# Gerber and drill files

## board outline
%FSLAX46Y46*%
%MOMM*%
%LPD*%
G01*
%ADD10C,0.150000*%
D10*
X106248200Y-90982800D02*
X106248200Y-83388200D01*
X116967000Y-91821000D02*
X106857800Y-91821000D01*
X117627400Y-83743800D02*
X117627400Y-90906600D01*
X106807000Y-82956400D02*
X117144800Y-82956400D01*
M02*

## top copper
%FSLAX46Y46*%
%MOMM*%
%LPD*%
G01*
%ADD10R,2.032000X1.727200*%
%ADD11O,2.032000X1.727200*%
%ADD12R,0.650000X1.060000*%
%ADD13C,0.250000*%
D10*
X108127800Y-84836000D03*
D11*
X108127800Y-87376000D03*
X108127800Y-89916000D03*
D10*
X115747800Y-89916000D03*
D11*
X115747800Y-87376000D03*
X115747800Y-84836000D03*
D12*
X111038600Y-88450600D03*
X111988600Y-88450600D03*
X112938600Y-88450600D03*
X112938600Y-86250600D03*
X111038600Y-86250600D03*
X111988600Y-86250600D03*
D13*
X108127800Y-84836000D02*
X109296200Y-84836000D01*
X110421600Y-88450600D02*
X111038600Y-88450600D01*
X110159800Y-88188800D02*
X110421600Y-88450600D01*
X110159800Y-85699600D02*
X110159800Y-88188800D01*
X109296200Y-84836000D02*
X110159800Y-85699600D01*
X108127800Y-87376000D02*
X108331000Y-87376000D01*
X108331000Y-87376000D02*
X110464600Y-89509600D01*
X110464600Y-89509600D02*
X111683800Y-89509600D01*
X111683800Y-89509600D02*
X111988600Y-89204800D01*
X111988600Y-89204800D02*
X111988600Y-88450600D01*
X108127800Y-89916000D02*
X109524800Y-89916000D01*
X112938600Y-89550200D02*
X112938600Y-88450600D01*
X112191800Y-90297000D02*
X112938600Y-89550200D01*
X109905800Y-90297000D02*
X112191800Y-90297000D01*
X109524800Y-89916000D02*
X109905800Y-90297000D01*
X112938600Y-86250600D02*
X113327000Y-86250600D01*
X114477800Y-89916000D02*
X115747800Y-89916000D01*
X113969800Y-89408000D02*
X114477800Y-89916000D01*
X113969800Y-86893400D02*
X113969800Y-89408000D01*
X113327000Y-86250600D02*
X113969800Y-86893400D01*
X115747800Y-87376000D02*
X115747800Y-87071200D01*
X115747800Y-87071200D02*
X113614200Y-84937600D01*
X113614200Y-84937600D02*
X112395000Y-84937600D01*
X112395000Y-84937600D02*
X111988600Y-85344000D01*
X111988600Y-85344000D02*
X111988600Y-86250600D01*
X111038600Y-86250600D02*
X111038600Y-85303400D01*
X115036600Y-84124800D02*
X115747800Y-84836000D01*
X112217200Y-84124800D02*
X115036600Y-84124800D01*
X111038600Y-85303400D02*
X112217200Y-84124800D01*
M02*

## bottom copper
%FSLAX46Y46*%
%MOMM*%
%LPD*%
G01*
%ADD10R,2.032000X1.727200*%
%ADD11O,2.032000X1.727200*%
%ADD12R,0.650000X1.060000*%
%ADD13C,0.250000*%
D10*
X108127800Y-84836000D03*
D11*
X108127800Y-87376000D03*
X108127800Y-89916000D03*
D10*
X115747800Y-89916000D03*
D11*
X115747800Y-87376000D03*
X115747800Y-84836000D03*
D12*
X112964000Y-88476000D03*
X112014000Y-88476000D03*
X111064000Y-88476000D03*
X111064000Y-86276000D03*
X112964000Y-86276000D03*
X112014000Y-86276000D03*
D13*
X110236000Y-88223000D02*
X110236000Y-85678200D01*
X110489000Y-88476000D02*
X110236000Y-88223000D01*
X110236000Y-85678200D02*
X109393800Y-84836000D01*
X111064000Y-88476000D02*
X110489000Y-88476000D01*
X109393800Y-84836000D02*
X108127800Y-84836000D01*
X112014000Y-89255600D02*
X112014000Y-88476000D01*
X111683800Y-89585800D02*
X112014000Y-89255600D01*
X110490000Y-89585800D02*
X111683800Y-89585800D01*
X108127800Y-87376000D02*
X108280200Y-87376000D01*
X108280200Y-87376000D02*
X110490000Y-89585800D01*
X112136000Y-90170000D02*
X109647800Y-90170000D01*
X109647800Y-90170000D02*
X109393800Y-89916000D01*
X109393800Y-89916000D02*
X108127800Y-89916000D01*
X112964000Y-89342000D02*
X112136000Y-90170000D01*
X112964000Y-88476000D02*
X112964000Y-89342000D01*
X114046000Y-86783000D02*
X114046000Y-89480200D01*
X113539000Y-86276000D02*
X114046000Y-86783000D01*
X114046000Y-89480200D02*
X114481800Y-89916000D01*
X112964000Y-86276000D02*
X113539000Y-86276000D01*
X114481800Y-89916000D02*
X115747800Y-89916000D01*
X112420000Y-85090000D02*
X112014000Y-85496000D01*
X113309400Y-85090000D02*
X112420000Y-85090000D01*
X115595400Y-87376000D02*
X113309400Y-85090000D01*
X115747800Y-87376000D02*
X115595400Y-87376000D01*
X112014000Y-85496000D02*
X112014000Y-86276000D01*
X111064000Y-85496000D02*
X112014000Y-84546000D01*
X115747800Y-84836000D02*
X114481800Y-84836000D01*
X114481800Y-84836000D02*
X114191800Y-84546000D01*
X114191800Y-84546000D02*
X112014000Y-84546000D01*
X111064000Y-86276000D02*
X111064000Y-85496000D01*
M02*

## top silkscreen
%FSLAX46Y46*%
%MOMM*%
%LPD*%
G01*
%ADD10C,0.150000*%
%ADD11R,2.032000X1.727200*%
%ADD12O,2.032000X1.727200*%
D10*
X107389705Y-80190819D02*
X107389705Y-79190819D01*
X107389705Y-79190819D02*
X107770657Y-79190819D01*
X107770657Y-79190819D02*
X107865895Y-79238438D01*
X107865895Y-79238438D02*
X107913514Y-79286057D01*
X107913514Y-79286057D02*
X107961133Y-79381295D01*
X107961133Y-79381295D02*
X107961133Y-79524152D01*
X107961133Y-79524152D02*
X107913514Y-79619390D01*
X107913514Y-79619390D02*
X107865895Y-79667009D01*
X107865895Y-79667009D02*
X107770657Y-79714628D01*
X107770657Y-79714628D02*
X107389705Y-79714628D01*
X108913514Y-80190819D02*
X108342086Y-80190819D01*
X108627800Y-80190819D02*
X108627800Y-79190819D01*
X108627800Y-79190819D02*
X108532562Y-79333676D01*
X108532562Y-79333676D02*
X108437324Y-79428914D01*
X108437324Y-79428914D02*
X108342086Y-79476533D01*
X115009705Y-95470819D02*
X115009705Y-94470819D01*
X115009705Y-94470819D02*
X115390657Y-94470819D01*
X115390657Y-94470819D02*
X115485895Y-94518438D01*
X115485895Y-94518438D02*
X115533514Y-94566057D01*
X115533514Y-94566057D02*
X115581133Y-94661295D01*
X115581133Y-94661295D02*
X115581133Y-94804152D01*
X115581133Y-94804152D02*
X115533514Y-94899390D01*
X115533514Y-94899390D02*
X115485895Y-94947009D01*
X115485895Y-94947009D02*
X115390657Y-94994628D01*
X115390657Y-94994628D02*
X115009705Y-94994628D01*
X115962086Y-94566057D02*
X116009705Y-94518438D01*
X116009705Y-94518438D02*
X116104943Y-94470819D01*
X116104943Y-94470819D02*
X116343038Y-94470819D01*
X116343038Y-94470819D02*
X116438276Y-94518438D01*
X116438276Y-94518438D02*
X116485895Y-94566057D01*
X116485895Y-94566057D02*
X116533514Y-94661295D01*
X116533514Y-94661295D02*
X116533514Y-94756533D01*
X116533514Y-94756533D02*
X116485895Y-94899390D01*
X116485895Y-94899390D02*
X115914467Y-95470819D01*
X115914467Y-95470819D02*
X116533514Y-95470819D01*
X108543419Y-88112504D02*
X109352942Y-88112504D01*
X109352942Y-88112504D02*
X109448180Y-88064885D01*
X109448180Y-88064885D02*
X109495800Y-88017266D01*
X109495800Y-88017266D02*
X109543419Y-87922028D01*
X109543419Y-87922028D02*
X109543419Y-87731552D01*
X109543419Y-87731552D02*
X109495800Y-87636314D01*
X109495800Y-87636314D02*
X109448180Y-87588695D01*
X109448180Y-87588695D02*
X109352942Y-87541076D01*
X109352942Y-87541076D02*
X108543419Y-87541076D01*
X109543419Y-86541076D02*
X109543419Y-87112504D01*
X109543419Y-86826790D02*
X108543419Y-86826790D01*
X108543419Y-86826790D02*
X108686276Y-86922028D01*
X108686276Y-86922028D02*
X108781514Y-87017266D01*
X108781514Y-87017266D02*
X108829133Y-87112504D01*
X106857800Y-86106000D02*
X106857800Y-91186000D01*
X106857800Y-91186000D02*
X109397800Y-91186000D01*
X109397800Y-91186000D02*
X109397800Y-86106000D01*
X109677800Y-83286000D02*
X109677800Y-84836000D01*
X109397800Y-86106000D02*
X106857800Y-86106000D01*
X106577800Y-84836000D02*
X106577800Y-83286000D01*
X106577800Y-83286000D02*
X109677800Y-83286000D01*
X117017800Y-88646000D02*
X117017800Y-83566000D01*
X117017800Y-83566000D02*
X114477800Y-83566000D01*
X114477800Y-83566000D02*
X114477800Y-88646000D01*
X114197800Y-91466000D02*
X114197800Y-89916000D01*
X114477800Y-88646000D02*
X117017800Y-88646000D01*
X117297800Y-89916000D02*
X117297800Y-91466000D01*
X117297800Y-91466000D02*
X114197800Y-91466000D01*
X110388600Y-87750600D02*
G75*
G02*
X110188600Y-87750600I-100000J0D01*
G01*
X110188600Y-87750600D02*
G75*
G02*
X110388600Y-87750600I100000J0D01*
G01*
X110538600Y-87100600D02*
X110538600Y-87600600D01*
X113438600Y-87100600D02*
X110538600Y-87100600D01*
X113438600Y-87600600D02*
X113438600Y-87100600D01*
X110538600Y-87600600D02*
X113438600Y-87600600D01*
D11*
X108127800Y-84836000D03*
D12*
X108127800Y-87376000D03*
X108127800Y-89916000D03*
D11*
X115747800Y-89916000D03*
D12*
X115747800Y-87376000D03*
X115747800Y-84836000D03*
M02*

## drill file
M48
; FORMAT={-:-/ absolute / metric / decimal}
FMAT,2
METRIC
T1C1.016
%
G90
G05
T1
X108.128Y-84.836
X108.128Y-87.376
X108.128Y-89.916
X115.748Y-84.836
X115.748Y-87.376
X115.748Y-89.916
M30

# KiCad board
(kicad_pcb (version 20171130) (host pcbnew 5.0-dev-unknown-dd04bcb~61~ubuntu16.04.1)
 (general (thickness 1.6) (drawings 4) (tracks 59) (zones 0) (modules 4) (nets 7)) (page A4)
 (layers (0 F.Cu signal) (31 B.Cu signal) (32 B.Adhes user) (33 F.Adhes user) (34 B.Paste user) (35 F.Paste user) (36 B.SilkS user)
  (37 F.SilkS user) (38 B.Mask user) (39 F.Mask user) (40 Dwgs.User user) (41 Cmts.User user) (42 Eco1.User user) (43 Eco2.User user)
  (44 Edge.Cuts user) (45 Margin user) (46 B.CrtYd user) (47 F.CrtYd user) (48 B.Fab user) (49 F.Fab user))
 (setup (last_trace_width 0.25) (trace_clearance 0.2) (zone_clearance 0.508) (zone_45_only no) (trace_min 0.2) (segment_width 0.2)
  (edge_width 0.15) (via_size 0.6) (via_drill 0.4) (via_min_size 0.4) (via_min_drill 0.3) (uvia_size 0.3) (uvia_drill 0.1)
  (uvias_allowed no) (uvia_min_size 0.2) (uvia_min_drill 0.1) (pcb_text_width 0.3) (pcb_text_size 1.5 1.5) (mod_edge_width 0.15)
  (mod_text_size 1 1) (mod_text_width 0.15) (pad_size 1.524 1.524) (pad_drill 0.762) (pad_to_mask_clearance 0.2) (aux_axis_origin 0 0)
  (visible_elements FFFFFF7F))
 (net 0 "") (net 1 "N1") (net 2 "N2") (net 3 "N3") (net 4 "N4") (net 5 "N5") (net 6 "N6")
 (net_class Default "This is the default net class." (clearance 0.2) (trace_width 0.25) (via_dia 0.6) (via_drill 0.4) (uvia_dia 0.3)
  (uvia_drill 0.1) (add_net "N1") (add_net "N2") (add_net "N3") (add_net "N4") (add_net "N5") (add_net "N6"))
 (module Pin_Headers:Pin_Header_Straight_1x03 (layer F.Cu) (at 108.1278 84.836)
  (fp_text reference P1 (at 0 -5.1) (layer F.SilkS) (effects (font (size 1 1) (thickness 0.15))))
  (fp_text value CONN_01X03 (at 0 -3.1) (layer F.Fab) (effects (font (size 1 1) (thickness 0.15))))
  (fp_line (start -1.27 1.27) (end -1.27 6.35) (layer F.SilkS) (width 0.15))
  (fp_line (start -1.27 6.35) (end 1.27 6.35) (layer F.SilkS) (width 0.15))
  (fp_line (start 1.27 6.35) (end 1.27 1.27) (layer F.SilkS) (width 0.15))
  (fp_line (start 1.55 -1.55) (end 1.55 0) (layer F.SilkS) (width 0.15))
  (fp_line (start 1.27 1.27) (end -1.27 1.27) (layer F.SilkS) (width 0.15))
  (fp_line (start -1.55 0) (end -1.55 -1.55) (layer F.SilkS) (width 0.15))
  (fp_line (start -1.55 -1.55) (end 1.55 -1.55) (layer F.SilkS) (width 0.15))
  (pad 1 thru_hole rect (at 0 0) (size 2.032 1.7272) (drill 1.016) (layers *.Cu *.Mask F.SilkS) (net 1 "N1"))
  (pad 2 thru_hole oval (at 0 2.54) (size 2.032 1.7272) (drill 1.016) (layers *.Cu *.Mask F.SilkS) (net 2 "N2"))
  (pad 3 thru_hole oval (at 0 5.08) (size 2.032 1.7272) (drill 1.016) (layers *.Cu *.Mask F.SilkS) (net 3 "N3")))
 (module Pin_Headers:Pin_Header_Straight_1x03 (layer F.Cu) (at 115.7478 89.916 180)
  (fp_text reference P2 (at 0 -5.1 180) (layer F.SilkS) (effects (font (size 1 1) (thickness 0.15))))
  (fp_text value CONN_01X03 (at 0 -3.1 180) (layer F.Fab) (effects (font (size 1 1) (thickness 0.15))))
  (fp_line (start -1.27 1.27) (end -1.27 6.35) (layer F.SilkS) (width 0.15))
  (fp_line (start -1.27 6.35) (end 1.27 6.35) (layer F.SilkS) (width 0.15))
  (fp_line (start 1.27 6.35) (end 1.27 1.27) (layer F.SilkS) (width 0.15))
  (fp_line (start 1.55 -1.55) (end 1.55 0) (layer F.SilkS) (width 0.15))
  (fp_line (start 1.27 1.27) (end -1.27 1.27) (layer F.SilkS) (width 0.15))
  (fp_line (start -1.55 0) (end -1.55 -1.55) (layer F.SilkS) (width 0.15))
  (fp_line (start -1.55 -1.55) (end 1.55 -1.55) (layer F.SilkS) (width 0.15))
  (pad 1 thru_hole rect (at 0 0 180) (size 2.032 1.7272) (drill 1.016) (layers *.Cu *.Mask F.SilkS) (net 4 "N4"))
  (pad 2 thru_hole oval (at 0 2.54 180) (size 2.032 1.7272) (drill 1.016) (layers *.Cu *.Mask F.SilkS) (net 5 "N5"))
  (pad 3 thru_hole oval (at 0 5.08 180) (size 2.032 1.7272) (drill 1.016) (layers *.Cu *.Mask F.SilkS) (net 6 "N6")))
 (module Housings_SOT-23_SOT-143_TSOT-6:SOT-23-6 (layer F.Cu) (at 111.9886 87.3506 90)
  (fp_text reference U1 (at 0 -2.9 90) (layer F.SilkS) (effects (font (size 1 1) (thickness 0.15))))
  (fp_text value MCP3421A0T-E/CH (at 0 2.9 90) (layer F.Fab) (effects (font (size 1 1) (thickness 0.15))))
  (fp_circle (center -0.4 -1.7) (end -0.3 -1.7) (layer F.SilkS) (width 0.15))
  (fp_line (start 0.25 -1.45) (end -0.25 -1.45) (layer F.SilkS) (width 0.15))
  (fp_line (start 0.25 1.45) (end 0.25 -1.45) (layer F.SilkS) (width 0.15))
  (fp_line (start -0.25 1.45) (end 0.25 1.45) (layer F.SilkS) (width 0.15))
  (fp_line (start -0.25 -1.45) (end -0.25 1.45) (layer F.SilkS) (width 0.15))
  (pad 1 smd rect (at -1.1 -0.95 90) (size 1.06 0.65) (layers F.Cu F.Paste F.Mask) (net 1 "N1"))
  (pad 2 smd rect (at -1.1 0 90) (size 1.06 0.65) (layers F.Cu F.Paste F.Mask) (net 2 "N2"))
  (pad 3 smd rect (at -1.1 0.95 90) (size 1.06 0.65) (layers F.Cu F.Paste F.Mask) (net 3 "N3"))
  (pad 4 smd rect (at 1.1 0.95 90) (size 1.06 0.65) (layers F.Cu F.Paste F.Mask) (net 4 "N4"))
  (pad 6 smd rect (at 1.1 -0.95 90) (size 1.06 0.65) (layers F.Cu F.Paste F.Mask) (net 6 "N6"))
  (pad 5 smd rect (at 1.1 0 90) (size 1.06 0.65) (layers F.Cu F.Paste F.Mask) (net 5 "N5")))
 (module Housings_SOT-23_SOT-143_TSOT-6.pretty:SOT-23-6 (layer B.Cu) (at 112.014 87.376 90)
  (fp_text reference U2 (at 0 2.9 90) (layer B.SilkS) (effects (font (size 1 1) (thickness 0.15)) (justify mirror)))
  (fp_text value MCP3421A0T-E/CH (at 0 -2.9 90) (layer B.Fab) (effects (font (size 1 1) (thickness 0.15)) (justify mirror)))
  (pad 1 smd rect (at -1.1 0.95 90) (size 1.06 0.65) (layers B.Cu B.Paste B.Mask) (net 3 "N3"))
  (pad 2 smd rect (at -1.1 0 90) (size 1.06 0.65) (layers B.Cu B.Paste B.Mask) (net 2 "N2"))
  (pad 3 smd rect (at -1.1 -0.95 90) (size 1.06 0.65) (layers B.Cu B.Paste B.Mask) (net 1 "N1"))
  (pad 4 smd rect (at 1.1 -0.95 90) (size 1.06 0.65) (layers B.Cu B.Paste B.Mask) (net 6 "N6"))
  (pad 6 smd rect (at 1.1 0.95 90) (size 1.06 0.65) (layers B.Cu B.Paste B.Mask) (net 4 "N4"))
  (pad 5 smd rect (at 1.1 0 90) (size 1.06 0.65) (layers B.Cu B.Paste B.Mask) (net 5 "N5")))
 (gr_line (start 106.2482 90.9828) (end 106.2482 83.3882) (angle 90) (layer Edge.Cuts) (width 0.15))
 (gr_line (start 116.967 91.821) (end 106.8578 91.821) (angle 90) (layer Edge.Cuts) (width 0.15))
 (gr_line (start 117.6274 83.7438) (end 117.6274 90.9066) (angle 90) (layer Edge.Cuts) (width 0.15))
 (gr_line (start 106.807 82.9564) (end 117.1448 82.9564) (angle 90) (layer Edge.Cuts) (width 0.15))
 (segment (start 110.236 88.223) (end 110.236 85.6782) (width 0.25) (layer B.Cu) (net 1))
 (segment (start 110.489 88.476) (end 110.236 88.223) (width 0.25) (layer B.Cu) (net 1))
 (segment (start 110.236 85.6782) (end 109.3938 84.836) (width 0.25) (layer B.Cu) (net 1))
 (segment (start 111.064 88.476) (end 110.489 88.476) (width 0.25) (layer B.Cu) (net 1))
 (segment (start 109.3938 84.836) (end 108.1278 84.836) (width 0.25) (layer B.Cu) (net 1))
 (segment (start 108.1278 84.836) (end 109.2962 84.836) (width 0.25) (layer F.Cu) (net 1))
 (segment (start 110.4216 88.4506) (end 111.0386 88.4506) (width 0.25) (layer F.Cu) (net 1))
 (segment (start 110.1598 88.1888) (end 110.4216 88.4506) (width 0.25) (layer F.Cu) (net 1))
 (segment (start 110.1598 85.6996) (end 110.1598 88.1888) (width 0.25) (layer F.Cu) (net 1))
 (segment (start 109.2962 84.836) (end 110.1598 85.6996) (width 0.25) (layer F.Cu) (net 1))
 (segment (start 112.014 89.2556) (end 112.014 88.476) (width 0.25) (layer B.Cu) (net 2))
 (segment (start 111.6838 89.5858) (end 112.014 89.2556) (width 0.25) (layer B.Cu) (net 2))
 (segment (start 110.49 89.5858) (end 111.6838 89.5858) (width 0.25) (layer B.Cu) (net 2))
 (segment (start 108.1278 87.376) (end 108.2802 87.376) (width 0.25) (layer B.Cu) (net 2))
 (segment (start 108.2802 87.376) (end 110.49 89.5858) (width 0.25) (layer B.Cu) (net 2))
 (segment (start 108.1278 87.376) (end 108.331 87.376) (width 0.25) (layer F.Cu) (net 2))
 (segment (start 108.331 87.376) (end 110.4646 89.5096) (width 0.25) (layer F.Cu) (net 2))
 (segment (start 110.4646 89.5096) (end 111.6838 89.5096) (width 0.25) (layer F.Cu) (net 2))
 (segment (start 111.6838 89.5096) (end 111.9886 89.2048) (width 0.25) (layer F.Cu) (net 2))
 (segment (start 111.9886 89.2048) (end 111.9886 88.4506) (width 0.25) (layer F.Cu) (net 2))
 (segment (start 112.136 90.17) (end 109.6478 90.17) (width 0.25) (layer B.Cu) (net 3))
 (segment (start 109.6478 90.17) (end 109.3938 89.916) (width 0.25) (layer B.Cu) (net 3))
 (segment (start 109.3938 89.916) (end 108.1278 89.916) (width 0.25) (layer B.Cu) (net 3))
 (segment (start 112.964 89.342) (end 112.136 90.17) (width 0.25) (layer B.Cu) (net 3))
 (segment (start 112.964 88.476) (end 112.964 89.342) (width 0.25) (layer B.Cu) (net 3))
 (segment (start 108.1278 89.916) (end 109.5248 89.916) (width 0.25) (layer F.Cu) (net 3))
 (segment (start 112.9386 89.5502) (end 112.9386 88.4506) (width 0.25) (layer F.Cu) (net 3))
 (segment (start 112.1918 90.297) (end 112.9386 89.5502) (width 0.25) (layer F.Cu) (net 3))
 (segment (start 109.9058 90.297) (end 112.1918 90.297) (width 0.25) (layer F.Cu) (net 3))
 (segment (start 109.5248 89.916) (end 109.9058 90.297) (width 0.25) (layer F.Cu) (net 3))
 (segment (start 114.046 86.783) (end 114.046 89.4802) (width 0.25) (layer B.Cu) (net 4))
 (segment (start 113.539 86.276) (end 114.046 86.783) (width 0.25) (layer B.Cu) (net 4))
 (segment (start 114.046 89.4802) (end 114.4818 89.916) (width 0.25) (layer B.Cu) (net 4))
 (segment (start 112.964 86.276) (end 113.539 86.276) (width 0.25) (layer B.Cu) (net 4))
 (segment (start 114.4818 89.916) (end 115.7478 89.916) (width 0.25) (layer B.Cu) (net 4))
 (segment (start 112.9386 86.2506) (end 113.327 86.2506) (width 0.25) (layer F.Cu) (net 4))
 (segment (start 114.4778 89.916) (end 115.7478 89.916) (width 0.25) (layer F.Cu) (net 4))
 (segment (start 113.9698 89.408) (end 114.4778 89.916) (width 0.25) (layer F.Cu) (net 4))
 (segment (start 113.9698 86.8934) (end 113.9698 89.408) (width 0.25) (layer F.Cu) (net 4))
 (segment (start 113.327 86.2506) (end 113.9698 86.8934) (width 0.25) (layer F.Cu) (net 4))
 (segment (start 112.42 85.09) (end 112.014 85.496) (width 0.25) (layer B.Cu) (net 5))
 (segment (start 113.3094 85.09) (end 112.42 85.09) (width 0.25) (layer B.Cu) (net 5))
 (segment (start 115.5954 87.376) (end 113.3094 85.09) (width 0.25) (layer B.Cu) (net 5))
 (segment (start 115.7478 87.376) (end 115.5954 87.376) (width 0.25) (layer B.Cu) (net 5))
 (segment (start 112.014 85.496) (end 112.014 86.276) (width 0.25) (layer B.Cu) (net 5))
 (segment (start 115.7478 87.376) (end 115.7478 87.0712) (width 0.25) (layer F.Cu) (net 5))
 (segment (start 115.7478 87.0712) (end 113.6142 84.9376) (width 0.25) (layer F.Cu) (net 5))
 (segment (start 113.6142 84.9376) (end 112.395 84.9376) (width 0.25) (layer F.Cu) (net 5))
 (segment (start 112.395 84.9376) (end 111.9886 85.344) (width 0.25) (layer F.Cu) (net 5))
 (segment (start 111.9886 85.344) (end 111.9886 86.2506) (width 0.25) (layer F.Cu) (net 5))
 (segment (start 111.064 85.496) (end 112.014 84.546) (width 0.25) (layer B.Cu) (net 6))
 (segment (start 115.7478 84.836) (end 114.4818 84.836) (width 0.25) (layer B.Cu) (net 6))
 (segment (start 114.4818 84.836) (end 114.1918 84.546) (width 0.25) (layer B.Cu) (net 6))
 (segment (start 114.1918 84.546) (end 112.014 84.546) (width 0.25) (layer B.Cu) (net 6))
 (segment (start 111.064 86.276) (end 111.064 85.496) (width 0.25) (layer B.Cu) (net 6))
 (segment (start 111.0386 86.2506) (end 111.0386 85.3034) (width 0.25) (layer F.Cu) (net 6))
 (segment (start 115.0366 84.1248) (end 115.7478 84.836) (width 0.25) (layer F.Cu) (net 6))
 (segment (start 112.2172 84.1248) (end 115.0366 84.1248) (width 0.25) (layer F.Cu) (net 6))
 (segment (start 111.0386 85.3034) (end 112.2172 84.1248) (width 0.25) (layer F.Cu) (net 6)))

